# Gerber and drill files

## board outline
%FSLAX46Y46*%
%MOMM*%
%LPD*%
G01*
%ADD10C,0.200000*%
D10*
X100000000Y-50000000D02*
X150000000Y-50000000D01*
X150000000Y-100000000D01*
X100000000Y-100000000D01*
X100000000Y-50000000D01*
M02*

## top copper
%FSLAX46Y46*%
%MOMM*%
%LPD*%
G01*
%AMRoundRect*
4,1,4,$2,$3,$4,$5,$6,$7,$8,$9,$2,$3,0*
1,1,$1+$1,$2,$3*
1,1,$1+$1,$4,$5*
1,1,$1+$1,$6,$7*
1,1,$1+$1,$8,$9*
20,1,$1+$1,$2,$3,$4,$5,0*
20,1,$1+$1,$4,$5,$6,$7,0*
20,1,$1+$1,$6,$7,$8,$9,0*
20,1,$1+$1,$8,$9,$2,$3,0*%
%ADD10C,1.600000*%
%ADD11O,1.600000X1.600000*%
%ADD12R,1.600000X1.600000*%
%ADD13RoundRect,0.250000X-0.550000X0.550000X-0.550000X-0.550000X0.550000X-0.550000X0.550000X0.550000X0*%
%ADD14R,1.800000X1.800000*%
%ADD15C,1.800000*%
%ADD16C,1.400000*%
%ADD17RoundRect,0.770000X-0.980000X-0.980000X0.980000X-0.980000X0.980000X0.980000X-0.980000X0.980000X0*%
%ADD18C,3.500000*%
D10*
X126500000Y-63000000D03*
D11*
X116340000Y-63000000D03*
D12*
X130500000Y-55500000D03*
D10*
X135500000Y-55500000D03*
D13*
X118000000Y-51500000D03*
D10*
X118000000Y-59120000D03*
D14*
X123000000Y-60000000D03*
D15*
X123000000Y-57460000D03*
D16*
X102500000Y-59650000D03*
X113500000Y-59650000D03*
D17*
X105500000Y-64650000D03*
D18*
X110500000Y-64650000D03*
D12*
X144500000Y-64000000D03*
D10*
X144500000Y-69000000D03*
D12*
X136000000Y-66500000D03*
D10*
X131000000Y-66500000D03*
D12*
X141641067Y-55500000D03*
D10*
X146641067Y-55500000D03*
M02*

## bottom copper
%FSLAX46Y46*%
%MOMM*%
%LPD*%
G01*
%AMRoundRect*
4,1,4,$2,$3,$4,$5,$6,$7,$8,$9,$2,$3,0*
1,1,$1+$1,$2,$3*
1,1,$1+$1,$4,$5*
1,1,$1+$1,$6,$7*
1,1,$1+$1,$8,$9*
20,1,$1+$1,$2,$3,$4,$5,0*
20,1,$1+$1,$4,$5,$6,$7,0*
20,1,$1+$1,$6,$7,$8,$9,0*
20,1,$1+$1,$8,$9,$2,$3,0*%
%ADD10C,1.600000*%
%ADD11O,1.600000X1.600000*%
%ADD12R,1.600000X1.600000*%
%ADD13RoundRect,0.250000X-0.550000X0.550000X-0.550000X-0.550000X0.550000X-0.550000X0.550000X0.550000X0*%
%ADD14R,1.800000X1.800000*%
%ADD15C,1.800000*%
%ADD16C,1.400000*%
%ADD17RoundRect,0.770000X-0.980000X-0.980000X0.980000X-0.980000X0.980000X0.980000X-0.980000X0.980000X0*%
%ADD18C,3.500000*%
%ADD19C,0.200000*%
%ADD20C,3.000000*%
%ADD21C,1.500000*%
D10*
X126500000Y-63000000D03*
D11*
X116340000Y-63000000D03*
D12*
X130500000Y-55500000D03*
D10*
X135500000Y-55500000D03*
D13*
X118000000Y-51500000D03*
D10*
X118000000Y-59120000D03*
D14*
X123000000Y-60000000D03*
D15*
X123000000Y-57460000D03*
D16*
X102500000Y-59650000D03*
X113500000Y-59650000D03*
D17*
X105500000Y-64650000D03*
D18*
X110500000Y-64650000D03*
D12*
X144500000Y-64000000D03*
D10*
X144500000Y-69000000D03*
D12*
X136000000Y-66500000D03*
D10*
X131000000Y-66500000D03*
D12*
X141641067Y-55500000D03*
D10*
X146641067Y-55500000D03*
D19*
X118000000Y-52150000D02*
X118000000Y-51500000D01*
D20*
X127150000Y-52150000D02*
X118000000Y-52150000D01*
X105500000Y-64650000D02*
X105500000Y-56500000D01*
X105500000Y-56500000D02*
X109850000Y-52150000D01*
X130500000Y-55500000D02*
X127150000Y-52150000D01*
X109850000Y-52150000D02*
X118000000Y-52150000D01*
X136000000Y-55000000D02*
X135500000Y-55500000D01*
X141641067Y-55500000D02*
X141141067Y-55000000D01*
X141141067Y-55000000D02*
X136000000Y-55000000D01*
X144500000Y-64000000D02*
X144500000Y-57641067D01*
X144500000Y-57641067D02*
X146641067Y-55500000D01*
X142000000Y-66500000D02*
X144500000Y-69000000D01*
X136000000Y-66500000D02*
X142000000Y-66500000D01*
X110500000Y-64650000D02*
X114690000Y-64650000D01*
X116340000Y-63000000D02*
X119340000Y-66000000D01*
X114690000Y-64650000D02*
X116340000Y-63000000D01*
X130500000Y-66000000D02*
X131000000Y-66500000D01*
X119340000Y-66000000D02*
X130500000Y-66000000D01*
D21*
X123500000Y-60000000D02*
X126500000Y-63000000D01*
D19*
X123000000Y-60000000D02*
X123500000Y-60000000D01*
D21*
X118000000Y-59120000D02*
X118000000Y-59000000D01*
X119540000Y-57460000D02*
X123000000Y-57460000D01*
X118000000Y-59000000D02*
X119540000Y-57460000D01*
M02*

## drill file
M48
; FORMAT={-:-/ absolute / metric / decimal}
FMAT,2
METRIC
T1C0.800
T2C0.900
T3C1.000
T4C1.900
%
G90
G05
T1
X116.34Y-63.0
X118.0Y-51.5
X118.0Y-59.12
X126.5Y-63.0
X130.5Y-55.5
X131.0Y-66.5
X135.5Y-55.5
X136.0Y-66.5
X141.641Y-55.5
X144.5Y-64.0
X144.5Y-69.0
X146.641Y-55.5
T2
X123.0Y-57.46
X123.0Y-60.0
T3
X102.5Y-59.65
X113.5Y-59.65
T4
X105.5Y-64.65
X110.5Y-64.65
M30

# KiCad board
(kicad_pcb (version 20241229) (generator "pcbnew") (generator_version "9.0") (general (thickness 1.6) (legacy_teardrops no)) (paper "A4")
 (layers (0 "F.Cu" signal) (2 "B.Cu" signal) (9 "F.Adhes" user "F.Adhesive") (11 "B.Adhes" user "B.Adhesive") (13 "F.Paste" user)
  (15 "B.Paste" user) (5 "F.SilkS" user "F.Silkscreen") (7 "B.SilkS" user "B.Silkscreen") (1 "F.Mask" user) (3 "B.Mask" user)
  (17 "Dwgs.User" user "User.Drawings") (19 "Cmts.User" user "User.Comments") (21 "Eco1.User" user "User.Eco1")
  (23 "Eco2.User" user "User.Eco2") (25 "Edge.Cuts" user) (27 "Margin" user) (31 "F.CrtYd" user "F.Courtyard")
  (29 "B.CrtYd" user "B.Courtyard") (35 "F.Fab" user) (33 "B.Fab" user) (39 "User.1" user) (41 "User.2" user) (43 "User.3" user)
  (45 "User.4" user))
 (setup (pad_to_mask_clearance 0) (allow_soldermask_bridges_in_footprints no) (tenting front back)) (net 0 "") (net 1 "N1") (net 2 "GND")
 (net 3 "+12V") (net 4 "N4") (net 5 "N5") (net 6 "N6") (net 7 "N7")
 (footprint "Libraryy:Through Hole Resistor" (layer "F.Cu") (at 126.5 63 180)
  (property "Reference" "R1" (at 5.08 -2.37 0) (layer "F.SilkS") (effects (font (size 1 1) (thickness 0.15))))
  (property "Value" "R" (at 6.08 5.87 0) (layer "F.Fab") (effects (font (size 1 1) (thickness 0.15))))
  (pad "1" thru_hole circle (at 0 0 180) (size 1.6 1.6) (drill 0.8) (layers "*.Cu" "*.Mask") (remove_unused_layers no) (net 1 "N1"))
  (pad "2" thru_hole oval (at 10.16 0 180) (size 1.6 1.6) (drill 0.8) (layers "*.Cu" "*.Mask") (remove_unused_layers no) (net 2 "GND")))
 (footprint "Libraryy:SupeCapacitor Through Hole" (layer "F.Cu") (at 130.5 55.5)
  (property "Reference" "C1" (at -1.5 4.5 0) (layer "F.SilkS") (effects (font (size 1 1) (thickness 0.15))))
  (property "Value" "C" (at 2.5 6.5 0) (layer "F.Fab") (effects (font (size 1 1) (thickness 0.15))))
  (pad "1" thru_hole rect (at 0 0) (size 1.6 1.6) (drill 0.8) (layers "*.Cu" "*.Mask") (remove_unused_layers no) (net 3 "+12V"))
  (pad "2" thru_hole circle (at 5 0) (size 1.6 1.6) (drill 0.8) (layers "*.Cu" "*.Mask") (remove_unused_layers no) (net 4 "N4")))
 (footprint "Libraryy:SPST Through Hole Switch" (layer "F.Cu") (at 118 51.5 -90)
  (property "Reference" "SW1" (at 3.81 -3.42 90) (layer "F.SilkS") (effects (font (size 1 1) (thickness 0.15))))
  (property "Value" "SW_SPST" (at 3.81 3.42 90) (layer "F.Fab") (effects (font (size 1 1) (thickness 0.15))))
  (pad "1" thru_hole roundrect (at 0 0 270) (size 1.6 1.6) (drill 0.8) (layers "*.Cu" "*.Mask") (remove_unused_layers no)
   (roundrect_rratio 0.15625) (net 3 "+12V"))
  (pad "2" thru_hole circle (at 7.62 0 270) (size 1.6 1.6) (drill 0.8) (layers "*.Cu" "*.Mask") (remove_unused_layers no) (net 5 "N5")))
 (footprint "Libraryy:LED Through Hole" (layer "F.Cu") (at 123 60 90)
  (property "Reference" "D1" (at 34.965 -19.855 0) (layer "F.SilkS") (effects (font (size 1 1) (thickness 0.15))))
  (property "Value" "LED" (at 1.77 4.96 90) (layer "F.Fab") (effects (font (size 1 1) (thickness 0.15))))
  (pad "1" thru_hole rect (at 0 0 90) (size 1.8 1.8) (drill 0.9) (layers "*.Cu" "*.Mask") (remove_unused_layers no) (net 1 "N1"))
  (pad "2" thru_hole circle (at 2.54 0 90) (size 1.8 1.8) (drill 0.9) (layers "*.Cu" "*.Mask") (remove_unused_layers no) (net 5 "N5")))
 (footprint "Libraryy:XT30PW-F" (layer "F.Cu") (at 105.5 64.65)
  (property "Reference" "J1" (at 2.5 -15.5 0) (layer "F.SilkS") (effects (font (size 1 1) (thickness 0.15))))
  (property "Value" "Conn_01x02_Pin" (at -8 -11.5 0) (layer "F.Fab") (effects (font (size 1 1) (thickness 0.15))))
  (pad "" thru_hole circle (at -3 -5 90) (size 1.4 1.4) (drill 1) (layers "*.Cu" "*.Mask") (remove_unused_layers no))
  (pad "" thru_hole circle (at 8 -5) (size 1.4 1.4) (drill 1) (layers "*.Cu" "*.Mask") (remove_unused_layers no))
  (pad "1" thru_hole roundrect (at 0 0) (size 3.5 3.5) (drill 1.9) (layers "*.Cu" "*.Mask") (remove_unused_layers no)
   (roundrect_rratio 0.22) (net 3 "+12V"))
  (pad "2" thru_hole circle (at 5 0) (size 3.5 3.5) (drill 1.9) (layers "*.Cu" "*.Mask") (remove_unused_layers no) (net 2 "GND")))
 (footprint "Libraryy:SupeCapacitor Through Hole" (layer "F.Cu") (at 144.5 64 -90)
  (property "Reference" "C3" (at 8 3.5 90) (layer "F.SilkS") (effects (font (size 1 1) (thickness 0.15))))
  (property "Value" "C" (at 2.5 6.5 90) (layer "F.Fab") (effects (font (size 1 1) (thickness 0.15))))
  (pad "1" thru_hole rect (at 0 0 270) (size 1.6 1.6) (drill 0.8) (layers "*.Cu" "*.Mask") (remove_unused_layers no) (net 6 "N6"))
  (pad "2" thru_hole circle (at 5 0 270) (size 1.6 1.6) (drill 0.8) (layers "*.Cu" "*.Mask") (remove_unused_layers no) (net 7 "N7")))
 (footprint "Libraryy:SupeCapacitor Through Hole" (layer "F.Cu") (at 136 66.5 180)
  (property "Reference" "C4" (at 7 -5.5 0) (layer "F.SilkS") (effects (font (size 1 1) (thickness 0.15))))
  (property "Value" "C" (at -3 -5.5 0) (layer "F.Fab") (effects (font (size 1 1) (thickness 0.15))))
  (pad "1" thru_hole rect (at 0 0 180) (size 1.6 1.6) (drill 0.8) (layers "*.Cu" "*.Mask") (remove_unused_layers no) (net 7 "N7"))
  (pad "2" thru_hole circle (at 5 0 180) (size 1.6 1.6) (drill 0.8) (layers "*.Cu" "*.Mask") (remove_unused_layers no) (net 2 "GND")))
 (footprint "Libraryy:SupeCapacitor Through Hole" (layer "F.Cu") (at 141.641067 55.5)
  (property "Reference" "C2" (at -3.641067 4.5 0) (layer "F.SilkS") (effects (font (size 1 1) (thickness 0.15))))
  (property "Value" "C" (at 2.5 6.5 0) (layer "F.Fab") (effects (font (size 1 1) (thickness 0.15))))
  (pad "1" thru_hole rect (at 0 0) (size 1.6 1.6) (drill 0.8) (layers "*.Cu" "*.Mask") (remove_unused_layers no) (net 4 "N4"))
  (pad "2" thru_hole circle (at 5 0) (size 1.6 1.6) (drill 0.8) (layers "*.Cu" "*.Mask") (remove_unused_layers no) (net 6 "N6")))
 (gr_rect (start 100 50) (end 150 100) (stroke (width 0.2) (type solid)) (fill no) (layer "Edge.Cuts"))
 (segment (start 118 52.15) (end 118 51.5) (width 0.2) (layer "B.Cu") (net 3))
 (segment (start 127.15 52.15) (end 118 52.15) (width 3) (layer "B.Cu") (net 3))
 (segment (start 105.5 64.65) (end 105.5 56.5) (width 3) (layer "B.Cu") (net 3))
 (segment (start 105.5 56.5) (end 109.85 52.15) (width 3) (layer "B.Cu") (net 3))
 (segment (start 130.5 55.5) (end 127.15 52.15) (width 3) (layer "B.Cu") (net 3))
 (segment (start 109.85 52.15) (end 118 52.15) (width 3) (layer "B.Cu") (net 3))
 (segment (start 136 55) (end 135.5 55.5) (width 3) (layer "B.Cu") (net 4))
 (segment (start 141.641067 55.5) (end 141.141067 55) (width 3) (layer "B.Cu") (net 4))
 (segment (start 141.141067 55) (end 136 55) (width 3) (layer "B.Cu") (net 4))
 (segment (start 144.5 64) (end 144.5 57.641067) (width 3) (layer "B.Cu") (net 6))
 (segment (start 144.5 57.641067) (end 146.641067 55.5) (width 3) (layer "B.Cu") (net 6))
 (segment (start 142 66.5) (end 144.5 69) (width 3) (layer "B.Cu") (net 7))
 (segment (start 136 66.5) (end 142 66.5) (width 3) (layer "B.Cu") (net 7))
 (segment (start 110.5 64.65) (end 114.69 64.65) (width 3) (layer "B.Cu") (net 2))
 (segment (start 116.34 63) (end 119.34 66) (width 3) (layer "B.Cu") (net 2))
 (segment (start 114.69 64.65) (end 116.34 63) (width 3) (layer "B.Cu") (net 2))
 (segment (start 130.5 66) (end 131 66.5) (width 3) (layer "B.Cu") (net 2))
 (segment (start 119.34 66) (end 130.5 66) (width 3) (layer "B.Cu") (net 2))
 (segment (start 123.5 60) (end 126.5 63) (width 1.5) (layer "B.Cu") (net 1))
 (segment (start 123 60) (end 123.5 60) (width 0.2) (layer "B.Cu") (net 1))
 (segment (start 118 59.12) (end 118 59) (width 1.5) (layer "B.Cu") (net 5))
 (segment (start 119.54 57.46) (end 123 57.46) (width 1.5) (layer "B.Cu") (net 5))
 (segment (start 118 59) (end 119.54 57.46) (width 1.5) (layer "B.Cu") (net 5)))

